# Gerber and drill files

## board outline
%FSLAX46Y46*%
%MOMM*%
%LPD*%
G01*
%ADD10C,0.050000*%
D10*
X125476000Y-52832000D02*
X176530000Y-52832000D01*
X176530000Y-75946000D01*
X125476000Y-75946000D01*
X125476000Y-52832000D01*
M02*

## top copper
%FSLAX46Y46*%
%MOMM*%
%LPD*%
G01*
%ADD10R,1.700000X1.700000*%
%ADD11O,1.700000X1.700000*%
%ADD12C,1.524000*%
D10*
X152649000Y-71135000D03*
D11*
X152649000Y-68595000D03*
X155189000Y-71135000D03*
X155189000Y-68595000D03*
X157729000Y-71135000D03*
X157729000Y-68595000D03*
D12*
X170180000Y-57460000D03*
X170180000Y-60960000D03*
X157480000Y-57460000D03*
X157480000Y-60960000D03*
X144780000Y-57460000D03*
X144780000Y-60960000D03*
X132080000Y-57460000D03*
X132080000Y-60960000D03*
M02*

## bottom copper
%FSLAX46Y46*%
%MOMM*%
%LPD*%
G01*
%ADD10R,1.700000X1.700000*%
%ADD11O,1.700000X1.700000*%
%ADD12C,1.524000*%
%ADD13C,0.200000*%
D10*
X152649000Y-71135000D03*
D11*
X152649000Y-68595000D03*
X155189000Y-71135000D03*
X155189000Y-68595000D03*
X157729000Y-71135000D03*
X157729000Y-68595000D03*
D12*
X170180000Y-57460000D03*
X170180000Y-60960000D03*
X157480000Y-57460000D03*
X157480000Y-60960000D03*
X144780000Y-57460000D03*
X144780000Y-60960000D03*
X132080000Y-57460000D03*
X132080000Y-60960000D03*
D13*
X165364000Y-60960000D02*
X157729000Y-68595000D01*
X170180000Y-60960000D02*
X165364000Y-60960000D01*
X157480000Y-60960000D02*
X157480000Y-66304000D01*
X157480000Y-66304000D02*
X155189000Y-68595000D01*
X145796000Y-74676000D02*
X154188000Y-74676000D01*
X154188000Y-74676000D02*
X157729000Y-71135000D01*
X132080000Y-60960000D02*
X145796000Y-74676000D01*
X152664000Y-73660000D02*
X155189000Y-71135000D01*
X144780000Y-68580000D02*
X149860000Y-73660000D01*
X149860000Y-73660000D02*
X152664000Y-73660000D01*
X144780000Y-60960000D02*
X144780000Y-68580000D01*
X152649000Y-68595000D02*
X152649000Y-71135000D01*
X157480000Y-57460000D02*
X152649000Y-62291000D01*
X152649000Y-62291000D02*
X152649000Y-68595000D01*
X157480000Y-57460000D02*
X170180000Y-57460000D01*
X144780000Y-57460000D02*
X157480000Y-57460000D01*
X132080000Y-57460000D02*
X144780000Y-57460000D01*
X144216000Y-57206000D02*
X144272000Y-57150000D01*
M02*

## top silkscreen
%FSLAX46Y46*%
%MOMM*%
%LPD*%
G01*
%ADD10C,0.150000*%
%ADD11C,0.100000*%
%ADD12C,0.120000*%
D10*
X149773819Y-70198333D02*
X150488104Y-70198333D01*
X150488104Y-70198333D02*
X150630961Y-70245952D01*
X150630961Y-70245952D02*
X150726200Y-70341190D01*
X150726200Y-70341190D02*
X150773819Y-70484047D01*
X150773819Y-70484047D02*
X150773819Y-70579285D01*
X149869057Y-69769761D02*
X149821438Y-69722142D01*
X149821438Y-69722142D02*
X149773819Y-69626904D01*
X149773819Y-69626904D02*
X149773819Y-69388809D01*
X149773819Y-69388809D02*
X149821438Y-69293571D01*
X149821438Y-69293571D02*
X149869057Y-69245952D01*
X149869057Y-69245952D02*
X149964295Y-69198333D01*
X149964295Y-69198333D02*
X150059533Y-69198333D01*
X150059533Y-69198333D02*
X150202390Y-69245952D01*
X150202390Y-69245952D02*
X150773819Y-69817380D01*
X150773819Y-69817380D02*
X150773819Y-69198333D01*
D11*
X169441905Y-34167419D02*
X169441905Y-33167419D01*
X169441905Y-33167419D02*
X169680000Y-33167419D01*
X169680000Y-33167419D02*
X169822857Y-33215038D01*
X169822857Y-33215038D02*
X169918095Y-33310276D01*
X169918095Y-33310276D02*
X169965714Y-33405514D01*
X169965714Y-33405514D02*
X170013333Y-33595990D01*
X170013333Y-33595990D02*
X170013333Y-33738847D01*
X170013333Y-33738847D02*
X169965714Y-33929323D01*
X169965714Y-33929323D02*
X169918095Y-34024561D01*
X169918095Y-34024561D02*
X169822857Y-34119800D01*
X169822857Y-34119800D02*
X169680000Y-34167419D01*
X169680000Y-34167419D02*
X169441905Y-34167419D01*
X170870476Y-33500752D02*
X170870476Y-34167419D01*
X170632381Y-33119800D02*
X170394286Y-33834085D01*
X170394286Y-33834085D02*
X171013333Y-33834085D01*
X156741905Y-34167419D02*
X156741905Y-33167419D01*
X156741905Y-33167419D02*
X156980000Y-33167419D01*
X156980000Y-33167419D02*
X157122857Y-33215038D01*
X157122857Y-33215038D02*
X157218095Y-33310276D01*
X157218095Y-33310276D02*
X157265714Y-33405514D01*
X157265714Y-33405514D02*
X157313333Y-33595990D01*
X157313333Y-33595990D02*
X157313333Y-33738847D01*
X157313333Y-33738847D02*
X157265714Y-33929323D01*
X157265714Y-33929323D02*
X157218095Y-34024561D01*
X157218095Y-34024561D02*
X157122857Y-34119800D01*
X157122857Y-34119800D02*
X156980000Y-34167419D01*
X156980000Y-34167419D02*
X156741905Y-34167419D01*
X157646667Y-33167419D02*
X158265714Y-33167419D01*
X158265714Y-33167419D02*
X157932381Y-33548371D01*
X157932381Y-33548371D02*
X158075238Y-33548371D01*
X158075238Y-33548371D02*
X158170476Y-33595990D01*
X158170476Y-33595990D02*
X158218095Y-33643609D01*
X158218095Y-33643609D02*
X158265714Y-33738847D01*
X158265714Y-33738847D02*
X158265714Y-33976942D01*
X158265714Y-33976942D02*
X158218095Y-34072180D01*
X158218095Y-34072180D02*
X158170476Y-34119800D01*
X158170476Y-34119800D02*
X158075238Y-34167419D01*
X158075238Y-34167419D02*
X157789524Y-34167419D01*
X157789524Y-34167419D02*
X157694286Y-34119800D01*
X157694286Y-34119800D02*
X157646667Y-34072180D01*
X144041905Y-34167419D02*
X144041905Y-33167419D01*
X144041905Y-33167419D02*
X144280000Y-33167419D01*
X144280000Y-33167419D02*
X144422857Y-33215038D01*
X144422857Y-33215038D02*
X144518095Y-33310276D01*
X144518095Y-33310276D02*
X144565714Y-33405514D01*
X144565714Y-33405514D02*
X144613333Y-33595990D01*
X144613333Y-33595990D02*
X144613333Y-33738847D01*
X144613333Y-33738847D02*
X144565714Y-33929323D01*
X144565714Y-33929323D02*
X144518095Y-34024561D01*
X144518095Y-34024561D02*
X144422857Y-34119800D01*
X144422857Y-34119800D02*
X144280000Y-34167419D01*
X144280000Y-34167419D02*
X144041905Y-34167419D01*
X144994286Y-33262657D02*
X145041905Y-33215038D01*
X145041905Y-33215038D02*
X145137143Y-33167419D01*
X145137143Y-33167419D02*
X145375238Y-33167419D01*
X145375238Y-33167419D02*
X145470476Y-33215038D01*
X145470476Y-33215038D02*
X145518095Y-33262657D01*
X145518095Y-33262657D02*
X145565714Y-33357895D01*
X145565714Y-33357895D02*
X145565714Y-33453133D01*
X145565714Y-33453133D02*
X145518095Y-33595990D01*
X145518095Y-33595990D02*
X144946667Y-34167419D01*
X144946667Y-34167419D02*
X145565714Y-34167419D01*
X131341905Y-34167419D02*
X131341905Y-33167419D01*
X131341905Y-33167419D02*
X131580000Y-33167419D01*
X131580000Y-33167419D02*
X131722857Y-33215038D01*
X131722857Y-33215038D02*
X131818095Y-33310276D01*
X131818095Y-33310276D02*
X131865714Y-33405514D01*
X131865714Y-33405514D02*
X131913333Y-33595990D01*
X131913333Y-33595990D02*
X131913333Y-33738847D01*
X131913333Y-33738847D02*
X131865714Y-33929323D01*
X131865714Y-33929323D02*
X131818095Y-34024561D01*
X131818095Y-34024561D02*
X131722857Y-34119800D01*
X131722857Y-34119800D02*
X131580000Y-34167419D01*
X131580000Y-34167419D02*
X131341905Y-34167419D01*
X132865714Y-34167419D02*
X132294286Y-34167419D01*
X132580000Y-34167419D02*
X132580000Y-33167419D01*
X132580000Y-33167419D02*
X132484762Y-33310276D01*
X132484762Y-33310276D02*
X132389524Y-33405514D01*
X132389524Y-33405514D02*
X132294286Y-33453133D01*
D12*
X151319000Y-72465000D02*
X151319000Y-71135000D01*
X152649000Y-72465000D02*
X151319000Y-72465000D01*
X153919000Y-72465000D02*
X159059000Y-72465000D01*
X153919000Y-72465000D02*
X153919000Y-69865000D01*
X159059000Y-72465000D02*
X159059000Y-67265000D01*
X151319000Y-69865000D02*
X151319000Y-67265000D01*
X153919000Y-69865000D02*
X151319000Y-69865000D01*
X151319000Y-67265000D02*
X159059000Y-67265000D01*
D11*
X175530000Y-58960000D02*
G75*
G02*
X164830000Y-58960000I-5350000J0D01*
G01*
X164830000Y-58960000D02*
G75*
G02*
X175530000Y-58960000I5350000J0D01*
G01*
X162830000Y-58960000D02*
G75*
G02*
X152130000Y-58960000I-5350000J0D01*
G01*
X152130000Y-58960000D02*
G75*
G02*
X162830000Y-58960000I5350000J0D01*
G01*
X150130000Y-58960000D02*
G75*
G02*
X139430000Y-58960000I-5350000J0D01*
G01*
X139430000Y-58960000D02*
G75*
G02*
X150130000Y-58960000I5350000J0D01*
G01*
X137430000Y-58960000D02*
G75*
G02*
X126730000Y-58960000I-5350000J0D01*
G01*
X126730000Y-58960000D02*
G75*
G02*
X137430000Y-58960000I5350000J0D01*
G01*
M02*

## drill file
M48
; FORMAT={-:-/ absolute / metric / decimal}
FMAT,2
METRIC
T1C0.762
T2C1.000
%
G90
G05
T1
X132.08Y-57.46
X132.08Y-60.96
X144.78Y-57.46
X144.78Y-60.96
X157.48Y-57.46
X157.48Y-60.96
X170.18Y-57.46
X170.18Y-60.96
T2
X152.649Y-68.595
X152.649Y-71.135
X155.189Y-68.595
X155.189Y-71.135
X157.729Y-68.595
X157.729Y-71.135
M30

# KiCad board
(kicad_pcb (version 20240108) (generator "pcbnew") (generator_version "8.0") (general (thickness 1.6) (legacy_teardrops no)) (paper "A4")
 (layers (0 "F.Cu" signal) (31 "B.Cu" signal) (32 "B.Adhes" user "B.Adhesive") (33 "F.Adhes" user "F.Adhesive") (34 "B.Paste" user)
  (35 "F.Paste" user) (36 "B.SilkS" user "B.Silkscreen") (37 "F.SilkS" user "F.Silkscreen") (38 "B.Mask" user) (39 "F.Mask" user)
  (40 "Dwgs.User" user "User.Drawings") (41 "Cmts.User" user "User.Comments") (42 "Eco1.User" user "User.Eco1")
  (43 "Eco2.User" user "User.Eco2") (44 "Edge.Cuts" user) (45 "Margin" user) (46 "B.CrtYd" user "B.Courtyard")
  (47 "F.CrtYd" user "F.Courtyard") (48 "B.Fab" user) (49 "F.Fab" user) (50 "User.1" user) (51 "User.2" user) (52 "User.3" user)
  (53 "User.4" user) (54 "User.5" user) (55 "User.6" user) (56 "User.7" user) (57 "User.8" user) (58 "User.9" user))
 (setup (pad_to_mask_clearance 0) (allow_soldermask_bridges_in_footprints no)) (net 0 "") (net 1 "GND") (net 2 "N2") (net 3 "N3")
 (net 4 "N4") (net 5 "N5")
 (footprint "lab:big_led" (layer "F.Cu") (at 170.18 34.21)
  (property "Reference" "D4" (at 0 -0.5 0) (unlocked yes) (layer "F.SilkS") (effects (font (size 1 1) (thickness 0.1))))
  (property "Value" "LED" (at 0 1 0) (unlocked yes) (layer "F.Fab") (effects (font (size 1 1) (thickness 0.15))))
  (fp_circle (center 0 24.75) (end 5.35 24.75) (stroke (width 0.1) (type default)) (fill none) (layer "F.SilkS"))
  (pad "1" thru_hole circle (at 0 23.25) (size 1.524 1.524) (drill 0.762) (layers "*.Cu" "*.Mask") (remove_unused_layers no) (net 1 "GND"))
  (pad "2" thru_hole circle (at 0 26.75) (size 1.524 1.524) (drill 0.762) (layers "*.Cu" "*.Mask") (remove_unused_layers no) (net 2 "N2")))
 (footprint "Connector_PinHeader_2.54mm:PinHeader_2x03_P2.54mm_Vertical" (layer "F.Cu") (at 152.649 71.135 90)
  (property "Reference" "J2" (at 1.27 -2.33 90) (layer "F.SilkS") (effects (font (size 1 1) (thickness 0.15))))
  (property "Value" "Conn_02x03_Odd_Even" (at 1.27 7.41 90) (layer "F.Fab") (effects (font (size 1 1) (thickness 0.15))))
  (fp_line (start 3.87 -1.33) (end 3.87 6.41) (stroke (width 0.12) (type solid)) (layer "F.SilkS"))
  (fp_line (start 1.27 -1.33) (end 3.87 -1.33) (stroke (width 0.12) (type solid)) (layer "F.SilkS"))
  (fp_line (start -1.33 -1.33) (end 0 -1.33) (stroke (width 0.12) (type solid)) (layer "F.SilkS"))
  (fp_line (start -1.33 0) (end -1.33 -1.33) (stroke (width 0.12) (type solid)) (layer "F.SilkS"))
  (fp_line (start 1.27 1.27) (end 1.27 -1.33) (stroke (width 0.12) (type solid)) (layer "F.SilkS"))
  (fp_line (start -1.33 1.27) (end 1.27 1.27) (stroke (width 0.12) (type solid)) (layer "F.SilkS"))
  (fp_line (start -1.33 1.27) (end -1.33 6.41) (stroke (width 0.12) (type solid)) (layer "F.SilkS"))
  (fp_line (start -1.33 6.41) (end 3.87 6.41) (stroke (width 0.12) (type solid)) (layer "F.SilkS"))
  (pad "1" thru_hole rect (at 0 0 90) (size 1.7 1.7) (drill 1) (layers "*.Cu" "*.Mask") (remove_unused_layers no) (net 1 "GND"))
  (pad "2" thru_hole oval (at 2.54 0 90) (size 1.7 1.7) (drill 1) (layers "*.Cu" "*.Mask") (remove_unused_layers no) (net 1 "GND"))
  (pad "3" thru_hole oval (at 0 2.54 90) (size 1.7 1.7) (drill 1) (layers "*.Cu" "*.Mask") (remove_unused_layers no) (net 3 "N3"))
  (pad "4" thru_hole oval (at 2.54 2.54 90) (size 1.7 1.7) (drill 1) (layers "*.Cu" "*.Mask") (remove_unused_layers no) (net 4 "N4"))
  (pad "5" thru_hole oval (at 0 5.08 90) (size 1.7 1.7) (drill 1) (layers "*.Cu" "*.Mask") (remove_unused_layers no) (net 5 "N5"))
  (pad "6" thru_hole oval (at 2.54 5.08 90) (size 1.7 1.7) (drill 1) (layers "*.Cu" "*.Mask") (remove_unused_layers no) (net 2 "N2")))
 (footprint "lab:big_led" (layer "F.Cu") (at 144.78 34.21)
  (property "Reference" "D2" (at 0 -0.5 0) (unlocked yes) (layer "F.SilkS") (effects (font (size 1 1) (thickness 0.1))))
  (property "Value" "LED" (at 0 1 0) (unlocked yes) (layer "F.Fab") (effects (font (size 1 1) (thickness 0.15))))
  (fp_circle (center 0 24.75) (end 5.35 24.75) (stroke (width 0.1) (type default)) (fill none) (layer "F.SilkS"))
  (pad "1" thru_hole circle (at 0 23.25) (size 1.524 1.524) (drill 0.762) (layers "*.Cu" "*.Mask") (remove_unused_layers no) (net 1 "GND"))
  (pad "2" thru_hole circle (at 0 26.75) (size 1.524 1.524) (drill 0.762) (layers "*.Cu" "*.Mask") (remove_unused_layers no) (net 3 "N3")))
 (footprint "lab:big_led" (layer "F.Cu") (at 157.48 34.21)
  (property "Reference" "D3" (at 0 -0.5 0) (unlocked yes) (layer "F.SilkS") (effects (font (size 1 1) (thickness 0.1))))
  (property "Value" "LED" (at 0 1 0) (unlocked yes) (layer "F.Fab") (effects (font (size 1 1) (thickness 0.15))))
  (fp_circle (center 0 24.75) (end 5.35 24.75) (stroke (width 0.1) (type default)) (fill none) (layer "F.SilkS"))
  (pad "1" thru_hole circle (at 0 23.25) (size 1.524 1.524) (drill 0.762) (layers "*.Cu" "*.Mask") (remove_unused_layers no) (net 1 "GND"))
  (pad "2" thru_hole circle (at 0 26.75) (size 1.524 1.524) (drill 0.762) (layers "*.Cu" "*.Mask") (remove_unused_layers no) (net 4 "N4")))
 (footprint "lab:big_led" (layer "F.Cu") (at 132.08 34.21)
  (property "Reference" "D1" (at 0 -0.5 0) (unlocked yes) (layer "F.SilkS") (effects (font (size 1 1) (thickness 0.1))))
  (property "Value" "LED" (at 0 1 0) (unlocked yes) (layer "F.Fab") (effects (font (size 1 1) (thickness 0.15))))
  (fp_circle (center 0 24.75) (end 5.35 24.75) (stroke (width 0.1) (type default)) (fill none) (layer "F.SilkS"))
  (pad "1" thru_hole circle (at 0 23.25) (size 1.524 1.524) (drill 0.762) (layers "*.Cu" "*.Mask") (remove_unused_layers no) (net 1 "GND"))
  (pad "2" thru_hole circle (at 0 26.75) (size 1.524 1.524) (drill 0.762) (layers "*.Cu" "*.Mask") (remove_unused_layers no) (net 5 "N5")))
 (gr_rect (start 125.476 52.832) (end 176.53 75.946) (stroke (width 0.05) (type default)) (fill none) (layer "Edge.Cuts"))
 (segment (start 132.08 57.46) (end 144.78 57.46) (width 0.2) (layer "B.Cu") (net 1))
 (segment (start 144.78 57.46) (end 157.48 57.46) (width 0.2) (layer "B.Cu") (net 1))
 (segment (start 152.649 62.291) (end 152.649 68.595) (width 0.2) (layer "B.Cu") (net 1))
 (segment (start 157.48 57.46) (end 170.18 57.46) (width 0.2) (layer "B.Cu") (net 1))
 (segment (start 144.216 57.206) (end 144.272 57.15) (width 0.2) (layer "B.Cu") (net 1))
 (segment (start 152.649 68.595) (end 152.649 71.135) (width 0.2) (layer "B.Cu") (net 1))
 (segment (start 157.48 57.46) (end 152.649 62.291) (width 0.2) (layer "B.Cu") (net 1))
 (segment (start 145.796 74.676) (end 154.188 74.676) (width 0.2) (layer "B.Cu") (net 5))
 (segment (start 132.08 60.96) (end 145.796 74.676) (width 0.2) (layer "B.Cu") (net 5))
 (segment (start 154.188 74.676) (end 157.729 71.135) (width 0.2) (layer "B.Cu") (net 5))
 (segment (start 152.664 73.66) (end 155.189 71.135) (width 0.2) (layer "B.Cu") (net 3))
 (segment (start 144.78 60.96) (end 144.78 68.58) (width 0.2) (layer "B.Cu") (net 3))
 (segment (start 144.78 68.58) (end 149.86 73.66) (width 0.2) (layer "B.Cu") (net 3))
 (segment (start 149.86 73.66) (end 152.664 73.66) (width 0.2) (layer "B.Cu") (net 3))
 (segment (start 157.48 66.304) (end 155.189 68.595) (width 0.2) (layer "B.Cu") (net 4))
 (segment (start 157.48 60.96) (end 157.48 66.304) (width 0.2) (layer "B.Cu") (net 4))
 (segment (start 165.364 60.96) (end 157.729 68.595) (width 0.2) (layer "B.Cu") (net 2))
 (segment (start 170.18 60.96) (end 165.364 60.96) (width 0.2) (layer "B.Cu") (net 2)))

